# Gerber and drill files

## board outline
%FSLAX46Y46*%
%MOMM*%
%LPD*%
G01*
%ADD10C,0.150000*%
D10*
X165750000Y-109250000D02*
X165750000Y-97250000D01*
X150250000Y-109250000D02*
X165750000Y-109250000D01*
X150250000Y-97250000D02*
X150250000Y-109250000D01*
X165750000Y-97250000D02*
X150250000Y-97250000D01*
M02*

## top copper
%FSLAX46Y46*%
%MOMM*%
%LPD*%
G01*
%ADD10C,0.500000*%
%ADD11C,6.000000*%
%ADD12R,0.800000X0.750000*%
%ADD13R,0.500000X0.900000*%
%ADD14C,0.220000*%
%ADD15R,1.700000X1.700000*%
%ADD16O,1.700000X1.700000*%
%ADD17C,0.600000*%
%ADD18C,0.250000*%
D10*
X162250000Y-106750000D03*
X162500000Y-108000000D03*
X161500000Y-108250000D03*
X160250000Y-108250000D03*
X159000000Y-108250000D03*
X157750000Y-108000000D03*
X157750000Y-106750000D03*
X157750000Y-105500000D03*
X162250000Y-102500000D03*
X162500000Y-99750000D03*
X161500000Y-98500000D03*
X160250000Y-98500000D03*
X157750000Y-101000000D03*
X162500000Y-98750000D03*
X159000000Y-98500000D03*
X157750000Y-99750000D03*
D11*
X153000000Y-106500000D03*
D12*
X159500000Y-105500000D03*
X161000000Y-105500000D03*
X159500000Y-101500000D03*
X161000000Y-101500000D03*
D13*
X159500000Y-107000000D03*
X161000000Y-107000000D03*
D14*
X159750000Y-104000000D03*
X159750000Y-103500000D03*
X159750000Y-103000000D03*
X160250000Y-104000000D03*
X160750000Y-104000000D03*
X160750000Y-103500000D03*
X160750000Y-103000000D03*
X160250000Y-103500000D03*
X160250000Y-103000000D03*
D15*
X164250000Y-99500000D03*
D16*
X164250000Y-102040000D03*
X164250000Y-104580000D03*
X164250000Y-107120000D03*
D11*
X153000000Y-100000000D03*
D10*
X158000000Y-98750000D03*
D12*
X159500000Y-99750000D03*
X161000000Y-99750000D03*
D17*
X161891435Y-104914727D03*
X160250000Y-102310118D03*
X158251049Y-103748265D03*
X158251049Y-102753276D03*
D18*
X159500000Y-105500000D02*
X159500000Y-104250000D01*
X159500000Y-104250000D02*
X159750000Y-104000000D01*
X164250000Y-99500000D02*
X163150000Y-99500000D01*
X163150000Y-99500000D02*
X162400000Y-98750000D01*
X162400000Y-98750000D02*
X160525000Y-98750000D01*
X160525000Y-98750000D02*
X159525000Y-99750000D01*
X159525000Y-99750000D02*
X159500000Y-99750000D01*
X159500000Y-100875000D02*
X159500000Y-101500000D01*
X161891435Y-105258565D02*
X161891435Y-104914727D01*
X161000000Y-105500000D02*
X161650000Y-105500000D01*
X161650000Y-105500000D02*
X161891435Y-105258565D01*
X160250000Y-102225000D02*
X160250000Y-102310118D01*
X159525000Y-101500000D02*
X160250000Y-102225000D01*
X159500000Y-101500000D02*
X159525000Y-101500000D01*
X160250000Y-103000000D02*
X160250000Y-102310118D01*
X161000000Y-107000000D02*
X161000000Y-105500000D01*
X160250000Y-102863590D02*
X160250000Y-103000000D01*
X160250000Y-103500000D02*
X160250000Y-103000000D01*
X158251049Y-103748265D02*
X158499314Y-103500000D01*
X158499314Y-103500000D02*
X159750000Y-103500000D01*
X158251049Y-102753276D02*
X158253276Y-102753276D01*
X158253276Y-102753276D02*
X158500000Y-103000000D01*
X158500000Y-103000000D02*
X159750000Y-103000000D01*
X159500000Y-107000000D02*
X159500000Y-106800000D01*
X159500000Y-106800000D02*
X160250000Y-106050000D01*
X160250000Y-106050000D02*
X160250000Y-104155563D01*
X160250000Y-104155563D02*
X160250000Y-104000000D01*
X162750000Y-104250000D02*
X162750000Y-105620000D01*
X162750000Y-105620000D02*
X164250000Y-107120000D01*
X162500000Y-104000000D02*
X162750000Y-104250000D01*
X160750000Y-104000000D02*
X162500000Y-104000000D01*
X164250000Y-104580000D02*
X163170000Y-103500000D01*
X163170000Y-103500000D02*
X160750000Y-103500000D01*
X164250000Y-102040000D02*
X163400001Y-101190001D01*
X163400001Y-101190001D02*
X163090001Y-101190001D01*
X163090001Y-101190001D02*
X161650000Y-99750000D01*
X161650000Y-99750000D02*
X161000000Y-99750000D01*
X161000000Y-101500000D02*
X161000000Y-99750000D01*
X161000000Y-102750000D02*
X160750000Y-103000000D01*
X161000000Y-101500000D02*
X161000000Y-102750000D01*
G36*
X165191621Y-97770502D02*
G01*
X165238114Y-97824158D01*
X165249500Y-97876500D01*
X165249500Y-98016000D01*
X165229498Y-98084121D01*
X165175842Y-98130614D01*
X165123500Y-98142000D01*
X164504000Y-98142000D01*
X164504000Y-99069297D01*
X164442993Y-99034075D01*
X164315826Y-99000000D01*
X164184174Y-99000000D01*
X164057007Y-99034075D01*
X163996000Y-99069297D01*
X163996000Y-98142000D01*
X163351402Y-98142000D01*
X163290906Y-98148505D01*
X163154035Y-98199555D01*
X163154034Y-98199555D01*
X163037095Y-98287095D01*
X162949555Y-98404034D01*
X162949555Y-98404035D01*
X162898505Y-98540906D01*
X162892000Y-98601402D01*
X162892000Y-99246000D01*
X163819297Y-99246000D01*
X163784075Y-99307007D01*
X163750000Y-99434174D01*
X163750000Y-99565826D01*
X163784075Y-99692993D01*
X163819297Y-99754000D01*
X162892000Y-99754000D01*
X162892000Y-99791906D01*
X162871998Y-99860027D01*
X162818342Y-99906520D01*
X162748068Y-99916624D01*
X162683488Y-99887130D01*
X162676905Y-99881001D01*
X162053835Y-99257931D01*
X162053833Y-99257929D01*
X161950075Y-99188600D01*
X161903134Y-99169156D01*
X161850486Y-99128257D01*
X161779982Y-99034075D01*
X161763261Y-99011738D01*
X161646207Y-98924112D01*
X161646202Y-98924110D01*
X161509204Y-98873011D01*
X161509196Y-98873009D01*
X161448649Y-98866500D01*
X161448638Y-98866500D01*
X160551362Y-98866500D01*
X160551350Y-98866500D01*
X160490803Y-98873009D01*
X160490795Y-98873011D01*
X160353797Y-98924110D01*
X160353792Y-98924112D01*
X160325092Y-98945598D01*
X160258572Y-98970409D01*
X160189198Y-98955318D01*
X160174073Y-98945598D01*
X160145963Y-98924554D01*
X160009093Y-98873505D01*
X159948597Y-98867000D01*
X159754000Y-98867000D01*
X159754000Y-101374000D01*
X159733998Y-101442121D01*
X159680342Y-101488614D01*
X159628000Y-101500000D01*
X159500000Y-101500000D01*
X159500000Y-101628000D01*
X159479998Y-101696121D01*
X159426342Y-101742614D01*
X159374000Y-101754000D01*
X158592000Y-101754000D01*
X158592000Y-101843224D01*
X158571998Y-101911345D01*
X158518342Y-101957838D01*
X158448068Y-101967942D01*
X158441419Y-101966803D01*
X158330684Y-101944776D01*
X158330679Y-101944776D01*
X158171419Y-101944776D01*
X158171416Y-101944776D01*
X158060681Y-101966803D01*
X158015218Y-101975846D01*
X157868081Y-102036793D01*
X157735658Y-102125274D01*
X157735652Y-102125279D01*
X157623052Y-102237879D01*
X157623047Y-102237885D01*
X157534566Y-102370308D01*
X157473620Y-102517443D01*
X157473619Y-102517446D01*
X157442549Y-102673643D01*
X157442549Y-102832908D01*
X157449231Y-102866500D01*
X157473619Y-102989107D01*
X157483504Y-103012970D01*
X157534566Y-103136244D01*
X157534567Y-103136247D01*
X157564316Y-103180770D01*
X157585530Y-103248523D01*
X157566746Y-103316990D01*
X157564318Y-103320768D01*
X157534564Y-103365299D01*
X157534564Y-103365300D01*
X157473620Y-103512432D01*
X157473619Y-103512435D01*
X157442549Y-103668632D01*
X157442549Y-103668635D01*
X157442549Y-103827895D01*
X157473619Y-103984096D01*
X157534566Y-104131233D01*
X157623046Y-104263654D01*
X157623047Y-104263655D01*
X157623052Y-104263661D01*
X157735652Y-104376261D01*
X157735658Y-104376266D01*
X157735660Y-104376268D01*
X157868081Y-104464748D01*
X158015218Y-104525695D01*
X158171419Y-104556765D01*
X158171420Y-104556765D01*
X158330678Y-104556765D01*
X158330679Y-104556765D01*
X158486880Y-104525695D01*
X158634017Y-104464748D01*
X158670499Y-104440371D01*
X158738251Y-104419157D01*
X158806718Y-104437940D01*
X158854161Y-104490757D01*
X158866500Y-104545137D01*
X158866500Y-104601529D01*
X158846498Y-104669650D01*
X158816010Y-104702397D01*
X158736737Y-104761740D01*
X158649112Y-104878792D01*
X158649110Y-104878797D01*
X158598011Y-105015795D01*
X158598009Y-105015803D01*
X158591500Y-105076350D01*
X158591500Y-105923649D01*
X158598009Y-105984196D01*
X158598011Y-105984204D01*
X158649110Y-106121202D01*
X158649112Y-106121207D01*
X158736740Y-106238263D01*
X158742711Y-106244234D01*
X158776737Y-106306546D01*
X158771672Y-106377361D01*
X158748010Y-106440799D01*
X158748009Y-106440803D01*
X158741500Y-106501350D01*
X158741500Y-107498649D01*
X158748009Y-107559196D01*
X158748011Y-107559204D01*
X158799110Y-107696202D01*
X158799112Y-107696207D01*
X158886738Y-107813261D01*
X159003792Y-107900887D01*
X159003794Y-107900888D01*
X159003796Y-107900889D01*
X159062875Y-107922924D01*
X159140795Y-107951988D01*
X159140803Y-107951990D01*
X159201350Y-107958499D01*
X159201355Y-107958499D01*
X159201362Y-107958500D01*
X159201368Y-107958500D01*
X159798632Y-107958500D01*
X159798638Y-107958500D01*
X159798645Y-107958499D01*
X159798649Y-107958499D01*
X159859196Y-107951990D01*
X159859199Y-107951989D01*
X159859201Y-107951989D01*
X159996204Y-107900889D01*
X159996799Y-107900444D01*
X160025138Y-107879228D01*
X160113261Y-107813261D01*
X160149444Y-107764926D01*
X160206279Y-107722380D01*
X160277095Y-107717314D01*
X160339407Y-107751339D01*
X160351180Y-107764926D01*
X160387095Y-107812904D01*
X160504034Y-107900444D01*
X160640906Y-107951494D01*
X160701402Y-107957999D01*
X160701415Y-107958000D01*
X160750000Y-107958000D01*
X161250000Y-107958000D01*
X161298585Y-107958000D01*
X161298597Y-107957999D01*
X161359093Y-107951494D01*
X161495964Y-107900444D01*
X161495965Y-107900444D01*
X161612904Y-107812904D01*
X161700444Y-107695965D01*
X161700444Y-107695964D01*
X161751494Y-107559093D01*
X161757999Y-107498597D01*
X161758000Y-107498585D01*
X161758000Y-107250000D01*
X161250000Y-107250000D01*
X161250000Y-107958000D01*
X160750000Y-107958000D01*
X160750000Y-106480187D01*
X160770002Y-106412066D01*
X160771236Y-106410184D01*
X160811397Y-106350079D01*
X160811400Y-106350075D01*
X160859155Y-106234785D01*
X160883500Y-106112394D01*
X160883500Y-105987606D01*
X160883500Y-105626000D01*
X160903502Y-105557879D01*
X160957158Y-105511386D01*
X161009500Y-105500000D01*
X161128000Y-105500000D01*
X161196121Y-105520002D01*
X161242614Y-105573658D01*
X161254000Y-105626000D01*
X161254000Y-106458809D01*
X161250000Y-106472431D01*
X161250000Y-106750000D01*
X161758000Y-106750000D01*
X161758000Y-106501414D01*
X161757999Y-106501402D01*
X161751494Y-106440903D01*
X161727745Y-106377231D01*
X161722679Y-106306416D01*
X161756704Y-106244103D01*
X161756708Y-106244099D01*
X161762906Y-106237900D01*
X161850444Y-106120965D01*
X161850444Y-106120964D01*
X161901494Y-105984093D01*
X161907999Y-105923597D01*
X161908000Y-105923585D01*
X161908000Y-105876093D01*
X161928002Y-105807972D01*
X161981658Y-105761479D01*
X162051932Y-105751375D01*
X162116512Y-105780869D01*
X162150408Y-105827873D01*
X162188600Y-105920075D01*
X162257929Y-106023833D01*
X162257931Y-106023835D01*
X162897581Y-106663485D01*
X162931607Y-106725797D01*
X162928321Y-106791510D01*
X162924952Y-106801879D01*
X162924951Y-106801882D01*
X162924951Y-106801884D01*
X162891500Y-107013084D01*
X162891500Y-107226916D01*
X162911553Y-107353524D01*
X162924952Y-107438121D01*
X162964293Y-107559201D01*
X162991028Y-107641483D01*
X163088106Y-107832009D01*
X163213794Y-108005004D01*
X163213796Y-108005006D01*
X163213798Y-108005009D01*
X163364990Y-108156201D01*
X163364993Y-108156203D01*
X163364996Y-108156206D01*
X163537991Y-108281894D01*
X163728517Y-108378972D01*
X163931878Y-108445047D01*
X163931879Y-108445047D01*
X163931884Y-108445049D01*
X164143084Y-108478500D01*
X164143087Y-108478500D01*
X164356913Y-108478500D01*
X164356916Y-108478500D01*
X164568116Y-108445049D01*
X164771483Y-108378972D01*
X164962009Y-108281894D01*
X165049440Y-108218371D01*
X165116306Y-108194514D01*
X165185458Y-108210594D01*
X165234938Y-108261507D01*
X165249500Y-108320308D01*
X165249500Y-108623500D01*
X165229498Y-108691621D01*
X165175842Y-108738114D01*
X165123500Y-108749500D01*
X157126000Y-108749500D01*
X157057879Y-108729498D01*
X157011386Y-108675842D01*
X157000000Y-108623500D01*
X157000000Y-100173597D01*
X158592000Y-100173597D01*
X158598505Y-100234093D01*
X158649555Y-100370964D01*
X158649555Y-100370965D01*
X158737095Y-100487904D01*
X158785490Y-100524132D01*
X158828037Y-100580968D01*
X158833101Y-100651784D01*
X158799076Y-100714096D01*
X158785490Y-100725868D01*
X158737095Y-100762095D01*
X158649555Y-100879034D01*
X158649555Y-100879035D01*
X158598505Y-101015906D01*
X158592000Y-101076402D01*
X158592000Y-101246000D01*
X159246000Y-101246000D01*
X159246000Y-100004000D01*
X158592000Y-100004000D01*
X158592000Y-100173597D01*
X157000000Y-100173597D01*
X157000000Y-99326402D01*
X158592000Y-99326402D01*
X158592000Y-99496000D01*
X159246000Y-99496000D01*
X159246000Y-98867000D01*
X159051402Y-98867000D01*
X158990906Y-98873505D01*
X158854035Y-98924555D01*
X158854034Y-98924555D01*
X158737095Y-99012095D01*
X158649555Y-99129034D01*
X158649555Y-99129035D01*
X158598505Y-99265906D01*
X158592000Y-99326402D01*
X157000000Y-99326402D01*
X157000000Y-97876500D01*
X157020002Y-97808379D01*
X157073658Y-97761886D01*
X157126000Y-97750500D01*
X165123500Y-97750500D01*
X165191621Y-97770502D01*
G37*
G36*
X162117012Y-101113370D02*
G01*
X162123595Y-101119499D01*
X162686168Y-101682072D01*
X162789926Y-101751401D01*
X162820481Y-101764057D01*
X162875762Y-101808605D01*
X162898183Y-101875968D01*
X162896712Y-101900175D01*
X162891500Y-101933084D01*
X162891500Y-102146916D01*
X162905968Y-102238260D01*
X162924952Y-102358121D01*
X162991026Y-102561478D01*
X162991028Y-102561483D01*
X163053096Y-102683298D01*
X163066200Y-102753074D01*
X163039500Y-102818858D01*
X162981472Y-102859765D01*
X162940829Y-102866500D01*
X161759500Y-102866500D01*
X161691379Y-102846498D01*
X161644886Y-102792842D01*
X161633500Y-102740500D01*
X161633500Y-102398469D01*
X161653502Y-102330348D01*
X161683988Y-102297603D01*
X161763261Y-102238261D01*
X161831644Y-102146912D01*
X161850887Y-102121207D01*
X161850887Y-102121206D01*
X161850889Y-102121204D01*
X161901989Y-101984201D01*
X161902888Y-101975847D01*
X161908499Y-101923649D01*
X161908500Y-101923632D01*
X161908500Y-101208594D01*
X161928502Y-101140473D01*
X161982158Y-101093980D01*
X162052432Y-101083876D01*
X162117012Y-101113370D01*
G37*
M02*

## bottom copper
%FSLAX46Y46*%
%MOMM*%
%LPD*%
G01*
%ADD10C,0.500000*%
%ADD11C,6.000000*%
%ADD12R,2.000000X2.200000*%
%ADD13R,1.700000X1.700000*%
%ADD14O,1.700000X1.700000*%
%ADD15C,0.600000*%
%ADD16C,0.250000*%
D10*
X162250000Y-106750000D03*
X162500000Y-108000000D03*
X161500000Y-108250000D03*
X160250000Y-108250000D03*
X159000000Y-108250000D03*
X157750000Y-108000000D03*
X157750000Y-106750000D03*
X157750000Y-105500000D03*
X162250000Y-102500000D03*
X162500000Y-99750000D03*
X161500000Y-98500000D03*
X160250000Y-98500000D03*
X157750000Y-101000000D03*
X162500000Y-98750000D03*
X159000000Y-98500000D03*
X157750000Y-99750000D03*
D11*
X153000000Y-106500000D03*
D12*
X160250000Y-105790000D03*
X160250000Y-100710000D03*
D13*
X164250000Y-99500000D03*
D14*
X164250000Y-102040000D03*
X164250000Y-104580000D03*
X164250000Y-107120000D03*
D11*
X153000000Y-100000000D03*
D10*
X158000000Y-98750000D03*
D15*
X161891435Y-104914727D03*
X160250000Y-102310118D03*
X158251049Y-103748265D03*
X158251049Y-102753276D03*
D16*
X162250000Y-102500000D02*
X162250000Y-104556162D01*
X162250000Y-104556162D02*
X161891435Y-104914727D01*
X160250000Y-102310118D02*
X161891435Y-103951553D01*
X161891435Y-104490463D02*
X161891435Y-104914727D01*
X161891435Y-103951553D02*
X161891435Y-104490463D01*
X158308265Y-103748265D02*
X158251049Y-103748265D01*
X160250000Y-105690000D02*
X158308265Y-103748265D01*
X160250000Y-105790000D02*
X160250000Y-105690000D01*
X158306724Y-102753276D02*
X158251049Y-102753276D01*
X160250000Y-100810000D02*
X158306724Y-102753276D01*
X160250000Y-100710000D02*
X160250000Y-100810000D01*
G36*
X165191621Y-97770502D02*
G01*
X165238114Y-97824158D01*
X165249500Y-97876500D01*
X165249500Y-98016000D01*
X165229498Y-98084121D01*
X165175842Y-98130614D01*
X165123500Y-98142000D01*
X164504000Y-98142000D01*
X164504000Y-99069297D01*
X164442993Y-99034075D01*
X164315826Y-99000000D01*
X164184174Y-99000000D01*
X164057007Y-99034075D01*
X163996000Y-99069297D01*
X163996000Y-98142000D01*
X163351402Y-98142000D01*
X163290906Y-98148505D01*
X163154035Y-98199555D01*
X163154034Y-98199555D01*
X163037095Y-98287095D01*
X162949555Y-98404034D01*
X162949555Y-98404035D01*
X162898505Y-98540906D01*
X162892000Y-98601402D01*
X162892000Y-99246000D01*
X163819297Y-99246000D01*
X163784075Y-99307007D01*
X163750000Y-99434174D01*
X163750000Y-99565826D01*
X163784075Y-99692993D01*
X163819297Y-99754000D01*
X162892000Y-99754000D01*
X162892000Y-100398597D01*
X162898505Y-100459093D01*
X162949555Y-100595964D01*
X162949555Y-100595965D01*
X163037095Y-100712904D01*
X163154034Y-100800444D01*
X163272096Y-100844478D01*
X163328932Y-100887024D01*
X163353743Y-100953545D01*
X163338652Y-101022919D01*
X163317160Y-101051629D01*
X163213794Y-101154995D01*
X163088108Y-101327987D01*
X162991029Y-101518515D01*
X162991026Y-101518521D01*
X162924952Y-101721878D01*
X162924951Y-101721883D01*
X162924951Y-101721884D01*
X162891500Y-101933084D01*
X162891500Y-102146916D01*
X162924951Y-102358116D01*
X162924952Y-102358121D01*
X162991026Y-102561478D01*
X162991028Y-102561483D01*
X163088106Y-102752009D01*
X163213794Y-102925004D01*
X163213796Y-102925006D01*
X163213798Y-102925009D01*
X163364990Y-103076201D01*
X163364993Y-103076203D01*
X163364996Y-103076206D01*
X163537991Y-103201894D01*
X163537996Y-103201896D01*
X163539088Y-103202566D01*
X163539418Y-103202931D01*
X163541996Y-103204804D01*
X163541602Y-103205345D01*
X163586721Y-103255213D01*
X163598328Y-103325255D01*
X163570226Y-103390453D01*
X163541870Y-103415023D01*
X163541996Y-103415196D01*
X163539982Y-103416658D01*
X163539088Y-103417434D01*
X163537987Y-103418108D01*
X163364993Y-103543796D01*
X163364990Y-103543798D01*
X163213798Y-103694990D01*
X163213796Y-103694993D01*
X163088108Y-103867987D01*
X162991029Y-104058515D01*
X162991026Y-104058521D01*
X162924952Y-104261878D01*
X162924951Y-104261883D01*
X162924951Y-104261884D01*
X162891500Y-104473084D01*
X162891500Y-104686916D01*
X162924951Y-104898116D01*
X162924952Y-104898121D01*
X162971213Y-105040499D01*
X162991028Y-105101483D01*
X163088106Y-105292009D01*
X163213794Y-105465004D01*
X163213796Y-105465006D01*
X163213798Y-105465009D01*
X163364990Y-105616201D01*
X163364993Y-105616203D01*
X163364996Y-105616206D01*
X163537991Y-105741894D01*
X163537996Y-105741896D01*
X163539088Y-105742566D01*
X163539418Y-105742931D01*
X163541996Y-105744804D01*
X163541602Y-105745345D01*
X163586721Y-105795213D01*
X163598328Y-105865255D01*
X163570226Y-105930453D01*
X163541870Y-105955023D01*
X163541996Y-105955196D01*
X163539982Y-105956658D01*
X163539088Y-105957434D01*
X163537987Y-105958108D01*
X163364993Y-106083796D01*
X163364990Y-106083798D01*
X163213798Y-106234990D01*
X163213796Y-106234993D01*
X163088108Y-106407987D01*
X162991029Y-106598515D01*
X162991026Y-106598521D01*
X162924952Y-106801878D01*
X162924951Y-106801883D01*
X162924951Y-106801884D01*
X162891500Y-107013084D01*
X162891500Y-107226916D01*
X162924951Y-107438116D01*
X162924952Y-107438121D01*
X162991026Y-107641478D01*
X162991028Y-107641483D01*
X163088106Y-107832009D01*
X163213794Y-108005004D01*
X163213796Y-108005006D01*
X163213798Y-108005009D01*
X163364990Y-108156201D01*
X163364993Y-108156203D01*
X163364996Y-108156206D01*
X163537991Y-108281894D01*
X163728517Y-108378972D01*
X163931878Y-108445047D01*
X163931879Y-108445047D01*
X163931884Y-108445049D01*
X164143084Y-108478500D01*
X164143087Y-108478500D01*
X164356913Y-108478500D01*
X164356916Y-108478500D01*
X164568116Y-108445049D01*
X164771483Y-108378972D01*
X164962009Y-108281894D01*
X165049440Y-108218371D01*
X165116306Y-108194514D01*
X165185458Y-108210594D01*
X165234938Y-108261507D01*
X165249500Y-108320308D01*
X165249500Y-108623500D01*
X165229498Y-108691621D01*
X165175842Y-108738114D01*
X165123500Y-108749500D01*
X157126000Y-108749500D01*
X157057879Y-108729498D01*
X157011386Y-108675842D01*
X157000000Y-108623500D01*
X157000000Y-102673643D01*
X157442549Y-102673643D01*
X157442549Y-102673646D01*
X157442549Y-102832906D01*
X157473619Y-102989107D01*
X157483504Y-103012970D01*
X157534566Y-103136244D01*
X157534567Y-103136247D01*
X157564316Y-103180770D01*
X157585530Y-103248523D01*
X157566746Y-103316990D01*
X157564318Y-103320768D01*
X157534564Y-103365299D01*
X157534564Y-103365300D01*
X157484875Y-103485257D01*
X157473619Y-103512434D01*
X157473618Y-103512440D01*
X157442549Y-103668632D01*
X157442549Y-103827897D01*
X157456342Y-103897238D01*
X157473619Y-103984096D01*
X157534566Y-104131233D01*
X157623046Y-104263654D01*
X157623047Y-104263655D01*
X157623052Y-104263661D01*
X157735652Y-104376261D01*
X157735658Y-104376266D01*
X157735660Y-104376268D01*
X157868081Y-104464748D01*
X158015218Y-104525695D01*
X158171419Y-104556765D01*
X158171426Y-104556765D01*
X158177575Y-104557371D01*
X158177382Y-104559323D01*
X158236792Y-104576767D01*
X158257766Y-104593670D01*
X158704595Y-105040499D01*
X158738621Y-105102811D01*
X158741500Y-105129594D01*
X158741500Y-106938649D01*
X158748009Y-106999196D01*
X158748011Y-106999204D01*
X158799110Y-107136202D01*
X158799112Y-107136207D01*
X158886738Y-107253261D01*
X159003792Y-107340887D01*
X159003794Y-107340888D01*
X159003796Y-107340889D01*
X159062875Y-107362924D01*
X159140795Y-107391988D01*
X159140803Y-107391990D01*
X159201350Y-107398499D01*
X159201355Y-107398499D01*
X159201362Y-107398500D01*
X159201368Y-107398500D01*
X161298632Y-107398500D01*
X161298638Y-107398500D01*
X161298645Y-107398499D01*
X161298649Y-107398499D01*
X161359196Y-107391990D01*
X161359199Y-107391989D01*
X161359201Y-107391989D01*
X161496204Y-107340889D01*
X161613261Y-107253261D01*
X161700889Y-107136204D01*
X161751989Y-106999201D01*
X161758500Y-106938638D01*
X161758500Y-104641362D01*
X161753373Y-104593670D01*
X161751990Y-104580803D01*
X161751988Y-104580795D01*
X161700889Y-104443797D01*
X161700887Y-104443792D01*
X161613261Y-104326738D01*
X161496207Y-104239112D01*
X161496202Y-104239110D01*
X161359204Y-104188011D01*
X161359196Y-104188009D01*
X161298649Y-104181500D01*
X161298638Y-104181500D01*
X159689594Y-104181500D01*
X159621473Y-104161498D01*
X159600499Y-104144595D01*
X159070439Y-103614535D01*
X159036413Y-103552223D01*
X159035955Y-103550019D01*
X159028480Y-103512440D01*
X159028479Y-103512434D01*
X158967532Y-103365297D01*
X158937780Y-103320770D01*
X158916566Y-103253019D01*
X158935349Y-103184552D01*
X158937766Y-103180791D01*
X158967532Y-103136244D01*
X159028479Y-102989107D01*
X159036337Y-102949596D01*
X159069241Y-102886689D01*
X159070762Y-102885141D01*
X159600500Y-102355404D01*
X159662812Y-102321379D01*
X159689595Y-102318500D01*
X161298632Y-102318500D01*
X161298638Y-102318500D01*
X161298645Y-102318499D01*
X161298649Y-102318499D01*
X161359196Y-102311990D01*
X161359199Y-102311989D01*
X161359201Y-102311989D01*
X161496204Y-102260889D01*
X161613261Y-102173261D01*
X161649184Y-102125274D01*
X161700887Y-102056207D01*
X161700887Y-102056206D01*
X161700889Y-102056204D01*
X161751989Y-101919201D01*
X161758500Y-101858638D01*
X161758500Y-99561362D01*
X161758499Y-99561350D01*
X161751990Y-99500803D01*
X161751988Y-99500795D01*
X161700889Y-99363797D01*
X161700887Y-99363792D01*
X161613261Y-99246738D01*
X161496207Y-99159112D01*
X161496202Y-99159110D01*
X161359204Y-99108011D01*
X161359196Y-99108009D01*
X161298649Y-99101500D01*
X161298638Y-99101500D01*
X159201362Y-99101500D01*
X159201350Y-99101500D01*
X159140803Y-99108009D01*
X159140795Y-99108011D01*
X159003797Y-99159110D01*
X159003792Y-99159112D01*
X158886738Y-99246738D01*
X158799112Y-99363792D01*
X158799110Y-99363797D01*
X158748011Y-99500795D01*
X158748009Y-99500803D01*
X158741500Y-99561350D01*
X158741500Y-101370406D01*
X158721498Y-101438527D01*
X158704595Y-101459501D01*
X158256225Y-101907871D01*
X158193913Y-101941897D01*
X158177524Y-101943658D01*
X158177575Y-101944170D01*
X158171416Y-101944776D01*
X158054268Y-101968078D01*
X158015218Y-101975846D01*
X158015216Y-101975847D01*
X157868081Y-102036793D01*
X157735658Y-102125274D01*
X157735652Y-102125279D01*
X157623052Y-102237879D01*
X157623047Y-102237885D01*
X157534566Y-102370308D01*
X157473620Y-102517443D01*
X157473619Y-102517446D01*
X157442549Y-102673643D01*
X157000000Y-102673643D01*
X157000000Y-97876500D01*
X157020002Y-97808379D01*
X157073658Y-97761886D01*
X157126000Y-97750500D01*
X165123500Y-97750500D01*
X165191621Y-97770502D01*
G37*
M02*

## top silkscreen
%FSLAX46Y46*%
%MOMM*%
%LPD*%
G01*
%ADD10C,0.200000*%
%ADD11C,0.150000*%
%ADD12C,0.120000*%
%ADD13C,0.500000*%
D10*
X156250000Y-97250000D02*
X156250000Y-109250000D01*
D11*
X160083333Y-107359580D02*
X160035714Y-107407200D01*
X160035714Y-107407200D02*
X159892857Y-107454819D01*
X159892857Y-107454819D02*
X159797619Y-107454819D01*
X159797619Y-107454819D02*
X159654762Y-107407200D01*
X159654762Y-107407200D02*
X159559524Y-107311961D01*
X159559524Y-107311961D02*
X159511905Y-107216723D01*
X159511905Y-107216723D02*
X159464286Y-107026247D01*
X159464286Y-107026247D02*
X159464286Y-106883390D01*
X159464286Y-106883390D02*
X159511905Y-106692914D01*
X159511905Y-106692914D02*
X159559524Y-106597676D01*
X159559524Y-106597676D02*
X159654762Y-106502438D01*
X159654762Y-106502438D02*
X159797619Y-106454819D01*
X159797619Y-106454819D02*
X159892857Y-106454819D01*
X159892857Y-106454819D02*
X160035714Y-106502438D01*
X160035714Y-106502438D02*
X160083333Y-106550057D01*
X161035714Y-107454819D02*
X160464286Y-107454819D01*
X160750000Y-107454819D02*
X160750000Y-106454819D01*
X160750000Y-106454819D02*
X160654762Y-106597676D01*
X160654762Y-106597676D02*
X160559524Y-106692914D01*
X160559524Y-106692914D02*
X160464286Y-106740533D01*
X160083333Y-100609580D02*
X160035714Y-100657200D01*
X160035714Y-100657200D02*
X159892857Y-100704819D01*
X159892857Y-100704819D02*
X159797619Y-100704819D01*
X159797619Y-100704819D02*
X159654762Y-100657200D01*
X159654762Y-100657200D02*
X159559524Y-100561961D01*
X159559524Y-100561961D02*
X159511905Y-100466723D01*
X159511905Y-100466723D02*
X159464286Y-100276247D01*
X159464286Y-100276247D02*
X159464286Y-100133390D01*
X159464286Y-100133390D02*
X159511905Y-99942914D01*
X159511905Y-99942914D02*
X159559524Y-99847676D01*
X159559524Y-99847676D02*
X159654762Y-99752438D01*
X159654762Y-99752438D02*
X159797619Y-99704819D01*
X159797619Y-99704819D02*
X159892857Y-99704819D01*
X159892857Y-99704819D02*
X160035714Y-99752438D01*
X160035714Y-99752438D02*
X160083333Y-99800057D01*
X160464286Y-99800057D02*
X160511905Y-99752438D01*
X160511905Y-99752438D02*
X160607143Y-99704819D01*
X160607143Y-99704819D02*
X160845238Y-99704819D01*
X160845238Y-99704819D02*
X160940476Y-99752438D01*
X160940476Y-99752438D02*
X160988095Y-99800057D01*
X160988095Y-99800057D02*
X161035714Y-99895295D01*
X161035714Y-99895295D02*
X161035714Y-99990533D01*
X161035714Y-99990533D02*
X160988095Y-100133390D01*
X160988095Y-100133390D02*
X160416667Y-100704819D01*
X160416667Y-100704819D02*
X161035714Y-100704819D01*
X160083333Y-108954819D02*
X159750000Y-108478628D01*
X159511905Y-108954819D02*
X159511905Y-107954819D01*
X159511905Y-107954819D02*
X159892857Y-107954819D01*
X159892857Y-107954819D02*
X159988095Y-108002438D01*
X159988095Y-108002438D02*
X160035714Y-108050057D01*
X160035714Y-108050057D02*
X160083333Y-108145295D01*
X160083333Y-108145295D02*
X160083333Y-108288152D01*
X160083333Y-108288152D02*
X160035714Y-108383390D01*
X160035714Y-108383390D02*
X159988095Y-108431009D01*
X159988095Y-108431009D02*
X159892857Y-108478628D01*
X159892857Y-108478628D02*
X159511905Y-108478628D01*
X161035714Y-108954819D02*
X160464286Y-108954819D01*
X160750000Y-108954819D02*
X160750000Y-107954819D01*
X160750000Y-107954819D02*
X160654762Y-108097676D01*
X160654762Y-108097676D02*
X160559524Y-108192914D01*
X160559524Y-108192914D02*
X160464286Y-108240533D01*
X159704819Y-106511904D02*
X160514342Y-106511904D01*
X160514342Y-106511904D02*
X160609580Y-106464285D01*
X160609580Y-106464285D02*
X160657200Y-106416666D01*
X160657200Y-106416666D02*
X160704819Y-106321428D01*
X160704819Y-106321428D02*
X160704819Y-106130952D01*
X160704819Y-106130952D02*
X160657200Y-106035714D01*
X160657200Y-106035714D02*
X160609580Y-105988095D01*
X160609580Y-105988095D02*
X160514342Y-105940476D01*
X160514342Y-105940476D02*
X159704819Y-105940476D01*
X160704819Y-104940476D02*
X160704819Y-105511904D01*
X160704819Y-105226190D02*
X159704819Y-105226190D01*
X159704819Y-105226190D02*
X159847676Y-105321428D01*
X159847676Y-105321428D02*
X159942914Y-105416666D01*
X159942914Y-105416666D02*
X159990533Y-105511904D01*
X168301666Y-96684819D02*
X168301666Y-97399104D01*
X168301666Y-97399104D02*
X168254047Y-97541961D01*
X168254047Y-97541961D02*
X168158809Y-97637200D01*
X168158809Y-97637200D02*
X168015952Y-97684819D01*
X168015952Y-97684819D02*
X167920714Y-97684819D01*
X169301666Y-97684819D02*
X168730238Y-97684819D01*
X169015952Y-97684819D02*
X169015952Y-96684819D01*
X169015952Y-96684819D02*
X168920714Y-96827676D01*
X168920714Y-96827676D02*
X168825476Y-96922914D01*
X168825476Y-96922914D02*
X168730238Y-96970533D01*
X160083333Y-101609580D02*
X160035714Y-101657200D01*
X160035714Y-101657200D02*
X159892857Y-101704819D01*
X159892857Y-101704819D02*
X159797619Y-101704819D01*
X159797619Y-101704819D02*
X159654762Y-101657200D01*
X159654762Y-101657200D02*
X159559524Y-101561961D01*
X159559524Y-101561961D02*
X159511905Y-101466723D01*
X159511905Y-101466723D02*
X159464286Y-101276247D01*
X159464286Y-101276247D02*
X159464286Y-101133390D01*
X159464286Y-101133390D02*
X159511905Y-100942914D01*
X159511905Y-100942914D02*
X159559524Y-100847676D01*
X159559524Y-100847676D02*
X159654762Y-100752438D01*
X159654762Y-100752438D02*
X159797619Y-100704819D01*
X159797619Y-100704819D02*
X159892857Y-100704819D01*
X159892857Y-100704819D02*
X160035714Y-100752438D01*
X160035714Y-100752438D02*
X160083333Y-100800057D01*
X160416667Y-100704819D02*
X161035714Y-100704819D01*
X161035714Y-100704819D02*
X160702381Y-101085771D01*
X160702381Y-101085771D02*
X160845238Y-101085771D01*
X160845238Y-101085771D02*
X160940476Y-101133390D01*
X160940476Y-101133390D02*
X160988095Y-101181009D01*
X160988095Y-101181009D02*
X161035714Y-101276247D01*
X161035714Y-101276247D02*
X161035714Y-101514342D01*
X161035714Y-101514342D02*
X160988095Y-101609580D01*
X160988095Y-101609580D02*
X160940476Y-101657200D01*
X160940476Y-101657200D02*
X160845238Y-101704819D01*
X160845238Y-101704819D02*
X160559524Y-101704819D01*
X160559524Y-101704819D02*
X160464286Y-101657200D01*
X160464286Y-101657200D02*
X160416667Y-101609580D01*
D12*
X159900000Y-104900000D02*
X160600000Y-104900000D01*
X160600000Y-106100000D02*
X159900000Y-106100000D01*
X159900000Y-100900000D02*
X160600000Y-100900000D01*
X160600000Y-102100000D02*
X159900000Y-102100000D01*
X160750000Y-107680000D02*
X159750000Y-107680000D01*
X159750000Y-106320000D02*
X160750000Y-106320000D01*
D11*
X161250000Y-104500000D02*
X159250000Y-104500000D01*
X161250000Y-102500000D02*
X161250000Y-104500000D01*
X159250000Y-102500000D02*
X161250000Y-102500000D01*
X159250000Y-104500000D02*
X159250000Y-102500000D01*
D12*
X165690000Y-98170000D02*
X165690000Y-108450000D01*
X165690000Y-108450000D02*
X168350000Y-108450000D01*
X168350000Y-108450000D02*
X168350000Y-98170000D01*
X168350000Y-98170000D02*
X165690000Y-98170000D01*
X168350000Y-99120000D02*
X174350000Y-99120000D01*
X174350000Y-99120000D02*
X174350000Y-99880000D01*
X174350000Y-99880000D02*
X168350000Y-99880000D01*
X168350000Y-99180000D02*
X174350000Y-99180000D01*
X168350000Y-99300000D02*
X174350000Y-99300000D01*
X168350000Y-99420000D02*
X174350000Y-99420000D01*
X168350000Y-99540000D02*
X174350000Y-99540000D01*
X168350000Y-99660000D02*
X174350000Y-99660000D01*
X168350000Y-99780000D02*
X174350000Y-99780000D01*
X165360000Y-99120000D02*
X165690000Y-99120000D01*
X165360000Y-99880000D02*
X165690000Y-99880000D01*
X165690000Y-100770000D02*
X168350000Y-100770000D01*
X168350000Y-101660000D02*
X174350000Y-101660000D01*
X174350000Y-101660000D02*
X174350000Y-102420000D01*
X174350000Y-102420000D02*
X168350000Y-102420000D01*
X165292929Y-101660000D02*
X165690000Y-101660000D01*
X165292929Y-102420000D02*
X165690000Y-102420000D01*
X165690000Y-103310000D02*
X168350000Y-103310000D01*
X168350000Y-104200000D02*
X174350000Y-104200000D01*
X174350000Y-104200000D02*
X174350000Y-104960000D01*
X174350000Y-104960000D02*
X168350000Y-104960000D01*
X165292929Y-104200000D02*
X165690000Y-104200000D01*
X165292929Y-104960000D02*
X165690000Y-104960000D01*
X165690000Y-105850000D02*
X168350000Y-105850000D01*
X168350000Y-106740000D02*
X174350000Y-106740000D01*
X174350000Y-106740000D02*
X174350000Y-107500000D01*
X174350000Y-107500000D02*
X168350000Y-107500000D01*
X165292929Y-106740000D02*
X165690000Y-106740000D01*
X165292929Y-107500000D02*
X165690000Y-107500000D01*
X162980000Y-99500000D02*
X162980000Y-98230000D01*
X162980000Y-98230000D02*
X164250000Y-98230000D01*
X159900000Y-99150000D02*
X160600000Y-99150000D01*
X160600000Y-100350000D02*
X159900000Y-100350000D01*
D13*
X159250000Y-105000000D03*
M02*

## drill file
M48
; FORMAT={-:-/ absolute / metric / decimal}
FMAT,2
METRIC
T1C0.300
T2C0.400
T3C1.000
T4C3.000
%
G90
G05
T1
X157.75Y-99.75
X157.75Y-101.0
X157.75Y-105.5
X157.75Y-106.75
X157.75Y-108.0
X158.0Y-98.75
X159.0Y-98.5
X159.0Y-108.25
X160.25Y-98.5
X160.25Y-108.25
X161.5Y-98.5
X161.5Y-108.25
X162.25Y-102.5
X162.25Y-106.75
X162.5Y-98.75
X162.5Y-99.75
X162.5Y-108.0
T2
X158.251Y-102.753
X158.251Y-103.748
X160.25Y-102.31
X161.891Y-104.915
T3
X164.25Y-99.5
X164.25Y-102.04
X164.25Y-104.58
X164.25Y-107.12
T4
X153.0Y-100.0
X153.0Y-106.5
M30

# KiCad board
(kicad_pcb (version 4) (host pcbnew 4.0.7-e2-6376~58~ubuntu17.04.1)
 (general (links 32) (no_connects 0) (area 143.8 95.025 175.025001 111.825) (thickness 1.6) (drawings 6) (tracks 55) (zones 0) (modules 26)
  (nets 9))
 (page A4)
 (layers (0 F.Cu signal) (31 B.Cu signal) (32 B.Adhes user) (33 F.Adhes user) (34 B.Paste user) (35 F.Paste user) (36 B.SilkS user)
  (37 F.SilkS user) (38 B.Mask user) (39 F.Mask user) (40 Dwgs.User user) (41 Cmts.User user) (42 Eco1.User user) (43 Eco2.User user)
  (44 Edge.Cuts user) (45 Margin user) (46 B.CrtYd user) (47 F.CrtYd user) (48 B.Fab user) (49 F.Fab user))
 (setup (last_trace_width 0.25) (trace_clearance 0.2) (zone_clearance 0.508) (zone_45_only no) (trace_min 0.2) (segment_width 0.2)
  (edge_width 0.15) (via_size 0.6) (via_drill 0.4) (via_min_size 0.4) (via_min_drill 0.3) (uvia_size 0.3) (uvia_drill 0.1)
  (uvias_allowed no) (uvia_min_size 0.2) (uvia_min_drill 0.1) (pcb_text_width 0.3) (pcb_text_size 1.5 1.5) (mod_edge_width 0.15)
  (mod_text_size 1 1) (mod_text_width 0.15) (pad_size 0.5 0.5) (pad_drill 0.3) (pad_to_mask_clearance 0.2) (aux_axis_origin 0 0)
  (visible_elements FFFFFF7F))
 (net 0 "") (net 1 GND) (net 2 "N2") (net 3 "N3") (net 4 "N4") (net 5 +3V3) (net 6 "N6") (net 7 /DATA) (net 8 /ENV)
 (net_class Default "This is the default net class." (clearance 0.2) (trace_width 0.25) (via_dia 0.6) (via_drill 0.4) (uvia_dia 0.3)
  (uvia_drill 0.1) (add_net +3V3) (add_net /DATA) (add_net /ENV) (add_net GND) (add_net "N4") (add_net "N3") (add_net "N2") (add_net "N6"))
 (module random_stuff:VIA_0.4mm (layer F.Cu) (at 162.25 106.75)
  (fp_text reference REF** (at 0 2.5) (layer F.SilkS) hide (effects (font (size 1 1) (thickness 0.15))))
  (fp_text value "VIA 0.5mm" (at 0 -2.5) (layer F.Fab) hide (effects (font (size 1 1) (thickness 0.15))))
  (pad 1 thru_hole circle (at 0 0) (size 0.5 0.5) (drill 0.3) (layers *.Cu) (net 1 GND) (zone_connect 2)))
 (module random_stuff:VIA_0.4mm (layer F.Cu) (at 162.5 108)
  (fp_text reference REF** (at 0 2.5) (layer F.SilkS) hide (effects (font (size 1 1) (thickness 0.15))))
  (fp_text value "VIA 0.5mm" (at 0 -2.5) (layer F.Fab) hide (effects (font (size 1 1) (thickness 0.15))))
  (pad 1 thru_hole circle (at 0 0) (size 0.5 0.5) (drill 0.3) (layers *.Cu) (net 1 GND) (zone_connect 2)))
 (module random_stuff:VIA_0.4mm (layer F.Cu) (at 161.5 108.25)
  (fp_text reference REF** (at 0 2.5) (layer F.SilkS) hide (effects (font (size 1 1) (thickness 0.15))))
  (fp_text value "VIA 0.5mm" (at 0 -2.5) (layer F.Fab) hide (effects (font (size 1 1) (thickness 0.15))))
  (pad 1 thru_hole circle (at 0 0) (size 0.5 0.5) (drill 0.3) (layers *.Cu) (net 1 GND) (zone_connect 2)))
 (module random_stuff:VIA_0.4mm (layer F.Cu) (at 160.25 108.25)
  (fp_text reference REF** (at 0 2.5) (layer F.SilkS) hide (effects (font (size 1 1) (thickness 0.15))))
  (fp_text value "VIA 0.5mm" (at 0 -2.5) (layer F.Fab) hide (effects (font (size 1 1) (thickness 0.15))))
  (pad 1 thru_hole circle (at 0 0) (size 0.5 0.5) (drill 0.3) (layers *.Cu) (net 1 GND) (zone_connect 2)))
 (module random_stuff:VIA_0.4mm (layer F.Cu) (at 159 108.25)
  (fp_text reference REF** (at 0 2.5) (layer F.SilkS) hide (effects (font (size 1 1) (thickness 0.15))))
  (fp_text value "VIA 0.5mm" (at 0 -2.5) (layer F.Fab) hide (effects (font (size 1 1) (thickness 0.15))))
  (pad 1 thru_hole circle (at 0 0) (size 0.5 0.5) (drill 0.3) (layers *.Cu) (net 1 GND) (zone_connect 2)))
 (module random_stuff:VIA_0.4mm (layer F.Cu) (at 157.75 108)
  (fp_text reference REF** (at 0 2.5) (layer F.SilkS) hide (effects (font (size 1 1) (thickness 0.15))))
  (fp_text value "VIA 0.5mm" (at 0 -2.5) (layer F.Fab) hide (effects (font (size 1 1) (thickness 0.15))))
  (pad 1 thru_hole circle (at 0 0) (size 0.5 0.5) (drill 0.3) (layers *.Cu) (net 1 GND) (zone_connect 2)))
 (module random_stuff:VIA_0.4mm (layer F.Cu) (at 157.75 106.75)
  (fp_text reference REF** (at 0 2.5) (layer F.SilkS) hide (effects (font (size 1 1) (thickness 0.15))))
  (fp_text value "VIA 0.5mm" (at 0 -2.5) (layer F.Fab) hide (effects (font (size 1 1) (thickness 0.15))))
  (pad 1 thru_hole circle (at 0 0) (size 0.5 0.5) (drill 0.3) (layers *.Cu) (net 1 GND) (zone_connect 2)))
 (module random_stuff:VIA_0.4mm (layer F.Cu) (at 157.75 105.5)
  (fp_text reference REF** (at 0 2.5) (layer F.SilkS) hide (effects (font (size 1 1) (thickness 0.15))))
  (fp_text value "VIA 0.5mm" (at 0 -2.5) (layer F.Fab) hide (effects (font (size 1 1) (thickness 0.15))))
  (pad 1 thru_hole circle (at 0 0) (size 0.5 0.5) (drill 0.3) (layers *.Cu) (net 1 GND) (zone_connect 2)))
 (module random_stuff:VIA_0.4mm (layer F.Cu) (at 162.25 102.5)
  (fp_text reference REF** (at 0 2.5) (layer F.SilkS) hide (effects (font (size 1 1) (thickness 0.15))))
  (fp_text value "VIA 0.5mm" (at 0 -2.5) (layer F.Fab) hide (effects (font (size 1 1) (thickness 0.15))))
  (pad 1 thru_hole circle (at 0 0) (size 0.5 0.5) (drill 0.3) (layers *.Cu) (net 1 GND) (zone_connect 2)))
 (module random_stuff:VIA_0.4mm (layer F.Cu) (at 162.5 99.75)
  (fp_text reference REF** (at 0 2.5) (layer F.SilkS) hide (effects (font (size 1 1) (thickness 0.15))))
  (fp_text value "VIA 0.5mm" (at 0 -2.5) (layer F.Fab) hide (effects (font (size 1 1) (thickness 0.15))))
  (pad 1 thru_hole circle (at 0 0) (size 0.5 0.5) (drill 0.3) (layers *.Cu) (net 1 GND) (zone_connect 2)))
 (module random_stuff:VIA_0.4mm (layer F.Cu) (at 161.5 98.5)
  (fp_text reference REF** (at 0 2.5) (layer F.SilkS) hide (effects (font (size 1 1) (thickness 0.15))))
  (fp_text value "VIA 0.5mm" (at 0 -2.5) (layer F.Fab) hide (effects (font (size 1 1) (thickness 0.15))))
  (pad 1 thru_hole circle (at 0 0) (size 0.5 0.5) (drill 0.3) (layers *.Cu) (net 1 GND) (zone_connect 2)))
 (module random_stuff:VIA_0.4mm (layer F.Cu) (at 160.25 98.5)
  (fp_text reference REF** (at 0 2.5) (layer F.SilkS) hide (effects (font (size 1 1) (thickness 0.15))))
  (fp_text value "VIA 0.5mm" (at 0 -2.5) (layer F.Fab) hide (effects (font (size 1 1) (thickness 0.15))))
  (pad 1 thru_hole circle (at 0 0) (size 0.5 0.5) (drill 0.3) (layers *.Cu) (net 1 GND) (zone_connect 2)))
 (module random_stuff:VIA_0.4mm (layer F.Cu) (at 157.75 101)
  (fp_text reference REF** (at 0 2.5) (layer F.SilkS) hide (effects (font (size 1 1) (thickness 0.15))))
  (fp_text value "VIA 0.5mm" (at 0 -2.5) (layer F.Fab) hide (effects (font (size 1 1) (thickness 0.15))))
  (pad 1 thru_hole circle (at 0 0) (size 0.5 0.5) (drill 0.3) (layers *.Cu) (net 1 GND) (zone_connect 2)))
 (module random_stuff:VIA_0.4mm (layer F.Cu) (at 162.5 98.75)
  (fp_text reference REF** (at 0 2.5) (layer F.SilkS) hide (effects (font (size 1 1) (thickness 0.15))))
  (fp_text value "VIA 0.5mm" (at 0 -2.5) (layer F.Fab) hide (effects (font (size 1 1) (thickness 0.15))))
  (pad 1 thru_hole circle (at 0 0) (size 0.5 0.5) (drill 0.3) (layers *.Cu) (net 1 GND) (zone_connect 2)))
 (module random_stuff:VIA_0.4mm (layer F.Cu) (at 159 98.5)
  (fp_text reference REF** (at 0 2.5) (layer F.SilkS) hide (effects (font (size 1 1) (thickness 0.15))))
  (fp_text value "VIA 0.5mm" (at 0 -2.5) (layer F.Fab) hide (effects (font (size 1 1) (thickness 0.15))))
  (pad 1 thru_hole circle (at 0 0) (size 0.5 0.5) (drill 0.3) (layers *.Cu) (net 1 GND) (zone_connect 2)))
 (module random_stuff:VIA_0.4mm (layer F.Cu) (at 157.75 99.75)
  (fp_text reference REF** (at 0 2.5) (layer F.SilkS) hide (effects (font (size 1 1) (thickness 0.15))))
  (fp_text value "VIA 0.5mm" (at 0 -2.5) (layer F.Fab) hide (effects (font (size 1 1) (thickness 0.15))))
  (pad 1 thru_hole circle (at 0 0) (size 0.5 0.5) (drill 0.3) (layers *.Cu) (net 1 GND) (zone_connect 2)))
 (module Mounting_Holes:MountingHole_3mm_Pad (layer F.Cu) (at 153 106.5)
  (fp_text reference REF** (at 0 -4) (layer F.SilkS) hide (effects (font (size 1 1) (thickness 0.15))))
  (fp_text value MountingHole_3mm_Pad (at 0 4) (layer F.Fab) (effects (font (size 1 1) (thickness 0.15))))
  (pad 1 thru_hole circle (at 0 0) (size 6 6) (drill 3) (layers *.Cu *.Mask)))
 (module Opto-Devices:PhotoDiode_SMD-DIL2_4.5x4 (layer B.Cu) (at 160.25 103.25 270)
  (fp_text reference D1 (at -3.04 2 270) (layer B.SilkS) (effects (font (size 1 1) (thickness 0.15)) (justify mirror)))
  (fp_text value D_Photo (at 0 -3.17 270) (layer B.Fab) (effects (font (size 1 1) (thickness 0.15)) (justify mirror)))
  (pad 2 smd rect (at 2.54 0 90) (size 2.2 2) (layers B.Cu B.Paste B.Mask) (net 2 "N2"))
  (pad 1 smd rect (at -2.54 0 90) (size 2.2 2) (layers B.Cu B.Paste B.Mask) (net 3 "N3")))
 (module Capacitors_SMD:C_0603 (layer F.Cu) (at 160.25 105.5 180)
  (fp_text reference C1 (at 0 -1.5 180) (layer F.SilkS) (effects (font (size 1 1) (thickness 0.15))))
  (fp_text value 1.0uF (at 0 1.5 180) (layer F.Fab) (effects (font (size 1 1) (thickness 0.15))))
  (fp_line (start 0.35 0.6) (end -0.35 0.6) (layer F.SilkS) (width 0.12))
  (fp_line (start -0.35 -0.6) (end 0.35 -0.6) (layer F.SilkS) (width 0.12))
  (pad 2 smd rect (at 0.75 0 180) (size 0.8 0.75) (layers F.Cu F.Paste F.Mask) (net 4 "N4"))
  (pad 1 smd rect (at -0.75 0 180) (size 0.8 0.75) (layers F.Cu F.Paste F.Mask) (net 1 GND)))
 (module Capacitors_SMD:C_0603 (layer F.Cu) (at 160.25 101.5 180)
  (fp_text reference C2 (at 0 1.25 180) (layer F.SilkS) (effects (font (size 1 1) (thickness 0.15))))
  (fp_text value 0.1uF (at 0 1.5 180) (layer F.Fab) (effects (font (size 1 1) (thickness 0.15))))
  (fp_line (start 0.35 0.6) (end -0.35 0.6) (layer F.SilkS) (width 0.12))
  (fp_line (start -0.35 -0.6) (end 0.35 -0.6) (layer F.SilkS) (width 0.12))
  (pad 2 smd rect (at 0.75 0 180) (size 0.8 0.75) (layers F.Cu F.Paste F.Mask) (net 1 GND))
  (pad 1 smd rect (at -0.75 0 180) (size 0.8 0.75) (layers F.Cu F.Paste F.Mask) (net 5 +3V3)))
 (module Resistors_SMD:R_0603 (layer F.Cu) (at 160.25 107)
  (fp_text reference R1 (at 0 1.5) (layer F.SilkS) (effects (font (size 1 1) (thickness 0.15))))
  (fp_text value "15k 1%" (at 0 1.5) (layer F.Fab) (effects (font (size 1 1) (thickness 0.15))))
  (fp_line (start 0.5 0.68) (end -0.5 0.68) (layer F.SilkS) (width 0.12))
  (fp_line (start -0.5 -0.68) (end 0.5 -0.68) (layer F.SilkS) (width 0.12))
  (pad 1 smd rect (at -0.75 0) (size 0.5 0.9) (layers F.Cu F.Paste F.Mask) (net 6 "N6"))
  (pad 2 smd rect (at 0.75 0) (size 0.5 0.9) (layers F.Cu F.Paste F.Mask) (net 1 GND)))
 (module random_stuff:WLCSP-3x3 (layer F.Cu) (at 160.25 103.5 90)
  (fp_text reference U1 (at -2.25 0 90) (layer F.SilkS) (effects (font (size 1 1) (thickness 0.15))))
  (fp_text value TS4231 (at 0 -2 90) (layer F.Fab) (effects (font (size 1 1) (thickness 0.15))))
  (fp_line (start -1 1) (end -1 -1) (layer F.SilkS) (width 0.15))
  (fp_line (start 1 1) (end -1 1) (layer F.SilkS) (width 0.15))
  (fp_line (start 1 -1) (end 1 1) (layer F.SilkS) (width 0.15))
  (fp_line (start -1 -1) (end 1 -1) (layer F.SilkS) (width 0.15))
  (pad A1 smd circle (at -0.5 -0.5 90) (size 0.22 0.22) (layers F.Cu F.Paste F.Mask) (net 4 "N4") (solder_mask_margin 0.05))
  (pad A2 smd circle (at 0 -0.5 90) (size 0.22 0.22) (layers F.Cu F.Paste F.Mask) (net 2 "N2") (solder_mask_margin 0.05))
  (pad A3 smd circle (at 0.5 -0.5 90) (size 0.22 0.22) (layers F.Cu F.Paste F.Mask) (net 3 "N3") (solder_mask_margin 0.05))
  (pad B1 smd circle (at -0.5 0 90) (size 0.22 0.22) (layers F.Cu F.Paste F.Mask) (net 6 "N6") (solder_mask_margin 0.05))
  (pad C1 smd circle (at -0.5 0.5 90) (size 0.22 0.22) (layers F.Cu F.Paste F.Mask) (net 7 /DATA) (solder_mask_margin 0.05))
  (pad C2 smd circle (at 0 0.5 90) (size 0.22 0.22) (layers F.Cu F.Paste F.Mask) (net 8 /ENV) (solder_mask_margin 0.05))
  (pad C3 smd circle (at 0.5 0.5 90) (size 0.22 0.22) (layers F.Cu F.Paste F.Mask) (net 5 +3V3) (solder_mask_margin 0.05))
  (pad B2 smd circle (at 0 0 90) (size 0.22 0.22) (layers F.Cu F.Paste F.Mask) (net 1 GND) (solder_mask_margin 0.05))
  (pad B3 smd circle (at 0.5 0 90) (size 0.22 0.22) (layers F.Cu F.Paste F.Mask) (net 1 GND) (solder_mask_margin 0.05))
  (pad "" smd circle (at -1.5 -1 90) (size 0.5 0.5) (layers F.SilkS)))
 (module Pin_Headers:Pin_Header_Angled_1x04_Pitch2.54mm (layer F.Cu) (at 164.25 99.5)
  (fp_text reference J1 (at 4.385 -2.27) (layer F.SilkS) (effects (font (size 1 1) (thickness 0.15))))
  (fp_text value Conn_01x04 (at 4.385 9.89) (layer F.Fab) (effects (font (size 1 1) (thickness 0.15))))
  (fp_line (start 1.44 -1.33) (end 1.44 8.95) (layer F.SilkS) (width 0.12))
  (fp_line (start 1.44 8.95) (end 4.1 8.95) (layer F.SilkS) (width 0.12))
  (fp_line (start 4.1 8.95) (end 4.1 -1.33) (layer F.SilkS) (width 0.12))
  (fp_line (start 4.1 -1.33) (end 1.44 -1.33) (layer F.SilkS) (width 0.12))
  (fp_line (start 4.1 -0.38) (end 10.1 -0.38) (layer F.SilkS) (width 0.12))
  (fp_line (start 10.1 -0.38) (end 10.1 0.38) (layer F.SilkS) (width 0.12))
  (fp_line (start 10.1 0.38) (end 4.1 0.38) (layer F.SilkS) (width 0.12))
  (fp_line (start 4.1 -0.32) (end 10.1 -0.32) (layer F.SilkS) (width 0.12))
  (fp_line (start 4.1 -0.2) (end 10.1 -0.2) (layer F.SilkS) (width 0.12))
  (fp_line (start 4.1 -0.08) (end 10.1 -0.08) (layer F.SilkS) (width 0.12))
  (fp_line (start 4.1 0.04) (end 10.1 0.04) (layer F.SilkS) (width 0.12))
  (fp_line (start 4.1 0.16) (end 10.1 0.16) (layer F.SilkS) (width 0.12))
  (fp_line (start 4.1 0.28) (end 10.1 0.28) (layer F.SilkS) (width 0.12))
  (fp_line (start 1.11 -0.38) (end 1.44 -0.38) (layer F.SilkS) (width 0.12))
  (fp_line (start 1.11 0.38) (end 1.44 0.38) (layer F.SilkS) (width 0.12))
  (fp_line (start 1.44 1.27) (end 4.1 1.27) (layer F.SilkS) (width 0.12))
  (fp_line (start 4.1 2.16) (end 10.1 2.16) (layer F.SilkS) (width 0.12))
  (fp_line (start 10.1 2.16) (end 10.1 2.92) (layer F.SilkS) (width 0.12))
  (fp_line (start 10.1 2.92) (end 4.1 2.92) (layer F.SilkS) (width 0.12))
  (fp_line (start 1.042929 2.16) (end 1.44 2.16) (layer F.SilkS) (width 0.12))
  (fp_line (start 1.042929 2.92) (end 1.44 2.92) (layer F.SilkS) (width 0.12))
  (fp_line (start 1.44 3.81) (end 4.1 3.81) (layer F.SilkS) (width 0.12))
  (fp_line (start 4.1 4.7) (end 10.1 4.7) (layer F.SilkS) (width 0.12))
  (fp_line (start 10.1 4.7) (end 10.1 5.46) (layer F.SilkS) (width 0.12))
  (fp_line (start 10.1 5.46) (end 4.1 5.46) (layer F.SilkS) (width 0.12))
  (fp_line (start 1.042929 4.7) (end 1.44 4.7) (layer F.SilkS) (width 0.12))
  (fp_line (start 1.042929 5.46) (end 1.44 5.46) (layer F.SilkS) (width 0.12))
  (fp_line (start 1.44 6.35) (end 4.1 6.35) (layer F.SilkS) (width 0.12))
  (fp_line (start 4.1 7.24) (end 10.1 7.24) (layer F.SilkS) (width 0.12))
  (fp_line (start 10.1 7.24) (end 10.1 8) (layer F.SilkS) (width 0.12))
  (fp_line (start 10.1 8) (end 4.1 8) (layer F.SilkS) (width 0.12))
  (fp_line (start 1.042929 7.24) (end 1.44 7.24) (layer F.SilkS) (width 0.12))
  (fp_line (start 1.042929 8) (end 1.44 8) (layer F.SilkS) (width 0.12))
  (fp_line (start -1.27 0) (end -1.27 -1.27) (layer F.SilkS) (width 0.12))
  (fp_line (start -1.27 -1.27) (end 0 -1.27) (layer F.SilkS) (width 0.12))
  (pad 1 thru_hole rect (at 0 0) (size 1.7 1.7) (drill 1) (layers *.Cu *.Mask) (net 1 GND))
  (pad 2 thru_hole oval (at 0 2.54) (size 1.7 1.7) (drill 1) (layers *.Cu *.Mask) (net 5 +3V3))
  (pad 3 thru_hole oval (at 0 5.08) (size 1.7 1.7) (drill 1) (layers *.Cu *.Mask) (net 8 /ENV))
  (pad 4 thru_hole oval (at 0 7.62) (size 1.7 1.7) (drill 1) (layers *.Cu *.Mask) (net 7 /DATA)))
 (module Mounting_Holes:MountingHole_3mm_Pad (layer F.Cu) (at 153 100)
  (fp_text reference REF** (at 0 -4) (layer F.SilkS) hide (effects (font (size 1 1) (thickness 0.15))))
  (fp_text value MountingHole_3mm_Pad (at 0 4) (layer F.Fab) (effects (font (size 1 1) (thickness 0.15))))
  (pad 1 thru_hole circle (at 0 0) (size 6 6) (drill 3) (layers *.Cu *.Mask)))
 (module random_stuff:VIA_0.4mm (layer F.Cu) (at 158 98.75)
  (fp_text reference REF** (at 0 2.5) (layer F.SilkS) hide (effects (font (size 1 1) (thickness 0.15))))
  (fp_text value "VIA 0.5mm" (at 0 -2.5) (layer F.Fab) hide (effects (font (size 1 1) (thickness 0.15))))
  (pad 1 thru_hole circle (at 0 0) (size 0.5 0.5) (drill 0.3) (layers *.Cu) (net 1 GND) (zone_connect 2)))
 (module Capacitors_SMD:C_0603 (layer F.Cu) (at 160.25 99.75 180)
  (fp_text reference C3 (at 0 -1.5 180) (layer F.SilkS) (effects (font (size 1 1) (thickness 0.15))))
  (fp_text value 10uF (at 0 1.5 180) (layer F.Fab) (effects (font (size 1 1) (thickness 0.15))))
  (fp_line (start 0.35 0.6) (end -0.35 0.6) (layer F.SilkS) (width 0.12))
  (fp_line (start -0.35 -0.6) (end 0.35 -0.6) (layer F.SilkS) (width 0.12))
  (pad 2 smd rect (at 0.75 0 180) (size 0.8 0.75) (layers F.Cu F.Paste F.Mask) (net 1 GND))
  (pad 1 smd rect (at -0.75 0 180) (size 0.8 0.75) (layers F.Cu F.Paste F.Mask) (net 5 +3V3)))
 (gr_line (start 156.25 97.25) (end 156.25 109.25) (layer F.SilkS) (width 0.2))
 (gr_line (start 165.75 109.25) (end 165.75 97.25) (layer Edge.Cuts) (width 0.15))
 (gr_line (start 150.25 109.25) (end 165.75 109.25) (layer Edge.Cuts) (width 0.15))
 (gr_line (start 150.25 97.25) (end 150.25 109.25) (layer Edge.Cuts) (width 0.15))
 (gr_line (start 165.75 97.25) (end 150.25 97.25) (layer Edge.Cuts) (width 0.15))
 (segment (start 159.5 105.5) (end 159.5 104.25) (width 0.25) (layer F.Cu) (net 4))
 (segment (start 159.5 104.25) (end 159.75 104) (width 0.25) (layer F.Cu) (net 4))
 (segment (start 162.25 102.5) (end 162.25 104.556162) (width 0.25) (layer B.Cu) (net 1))
 (segment (start 162.25 104.556162) (end 161.891435 104.914727) (width 0.25) (layer B.Cu) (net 1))
 (segment (start 164.25 99.5) (end 163.15 99.5) (width 0.25) (layer F.Cu) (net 1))
 (segment (start 163.15 99.5) (end 162.4 98.75) (width 0.25) (layer F.Cu) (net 1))
 (segment (start 162.4 98.75) (end 160.525 98.75) (width 0.25) (layer F.Cu) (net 1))
 (segment (start 160.525 98.75) (end 159.525 99.75) (width 0.25) (layer F.Cu) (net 1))
 (segment (start 159.525 99.75) (end 159.5 99.75) (width 0.25) (layer F.Cu) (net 1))
 (segment (start 159.5 100.875) (end 159.5 101.5) (width 0.25) (layer F.Cu) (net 1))
 (segment (start 161.891435 105.258565) (end 161.891435 104.914727) (width 0.25) (layer F.Cu) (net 1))
 (segment (start 161 105.5) (end 161.65 105.5) (width 0.25) (layer F.Cu) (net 1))
 (segment (start 161.65 105.5) (end 161.891435 105.258565) (width 0.25) (layer F.Cu) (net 1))
 (segment (start 160.25 102.310118) (end 161.891435 103.951553) (width 0.25) (layer B.Cu) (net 1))
 (via (at 161.891435 104.914727) (size 0.6) (drill 0.4) (layers F.Cu B.Cu) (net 1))
 (segment (start 161.891435 104.490463) (end 161.891435 104.914727) (width 0.25) (layer B.Cu) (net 1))
 (segment (start 161.891435 103.951553) (end 161.891435 104.490463) (width 0.25) (layer B.Cu) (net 1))
 (segment (start 160.25 102.225) (end 160.25 102.310118) (width 0.25) (layer F.Cu) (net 1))
 (segment (start 159.525 101.5) (end 160.25 102.225) (width 0.25) (layer F.Cu) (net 1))
 (segment (start 159.5 101.5) (end 159.525 101.5) (width 0.25) (layer F.Cu) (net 1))
 (via (at 160.25 102.310118) (size 0.6) (drill 0.4) (layers F.Cu B.Cu) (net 1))
 (segment (start 160.25 103) (end 160.25 102.310118) (width 0.25) (layer F.Cu) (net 1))
 (segment (start 161 107) (end 161 105.5) (width 0.25) (layer F.Cu) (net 1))
 (segment (start 160.25 102.86359) (end 160.25 103) (width 0.25) (layer F.Cu) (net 1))
 (segment (start 160.25 103.5) (end 160.25 103) (width 0.25) (layer F.Cu) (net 1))
 (segment (start 158.251049 103.748265) (end 158.499314 103.5) (width 0.25) (layer F.Cu) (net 2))
 (segment (start 158.499314 103.5) (end 159.75 103.5) (width 0.25) (layer F.Cu) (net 2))
 (segment (start 158.308265 103.748265) (end 158.251049 103.748265) (width 0.25) (layer B.Cu) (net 2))
 (segment (start 160.25 105.69) (end 158.308265 103.748265) (width 0.25) (layer B.Cu) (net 2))
 (segment (start 160.25 105.79) (end 160.25 105.69) (width 0.25) (layer B.Cu) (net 2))
 (via (at 158.251049 103.748265) (size 0.6) (drill 0.4) (layers F.Cu B.Cu) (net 2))
 (segment (start 158.251049 102.753276) (end 158.253276 102.753276) (width 0.25) (layer F.Cu) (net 3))
 (segment (start 158.253276 102.753276) (end 158.5 103) (width 0.25) (layer F.Cu) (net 3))
 (segment (start 158.5 103) (end 159.75 103) (width 0.25) (layer F.Cu) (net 3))
 (segment (start 158.306724 102.753276) (end 158.251049 102.753276) (width 0.25) (layer B.Cu) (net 3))
 (segment (start 160.25 100.81) (end 158.306724 102.753276) (width 0.25) (layer B.Cu) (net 3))
 (segment (start 160.25 100.71) (end 160.25 100.81) (width 0.25) (layer B.Cu) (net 3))
 (via (at 158.251049 102.753276) (size 0.6) (drill 0.4) (layers F.Cu B.Cu) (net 3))
 (segment (start 159.5 107) (end 159.5 106.8) (width 0.25) (layer F.Cu) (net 6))
 (segment (start 159.5 106.8) (end 160.25 106.05) (width 0.25) (layer F.Cu) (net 6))
 (segment (start 160.25 106.05) (end 160.25 104.155563) (width 0.25) (layer F.Cu) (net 6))
 (segment (start 160.25 104.155563) (end 160.25 104) (width 0.25) (layer F.Cu) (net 6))
 (segment (start 162.75 104.25) (end 162.75 105.62) (width 0.25) (layer F.Cu) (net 7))
 (segment (start 162.75 105.62) (end 164.25 107.12) (width 0.25) (layer F.Cu) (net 7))
 (segment (start 162.5 104) (end 162.75 104.25) (width 0.25) (layer F.Cu) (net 7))
 (segment (start 160.75 104) (end 162.5 104) (width 0.25) (layer F.Cu) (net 7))
 (segment (start 164.25 104.58) (end 163.17 103.5) (width 0.25) (layer F.Cu) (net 8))
 (segment (start 163.17 103.5) (end 160.75 103.5) (width 0.25) (layer F.Cu) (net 8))
 (segment (start 164.25 102.04) (end 163.400001 101.190001) (width 0.25) (layer F.Cu) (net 5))
 (segment (start 163.400001 101.190001) (end 163.090001 101.190001) (width 0.25) (layer F.Cu) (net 5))
 (segment (start 163.090001 101.190001) (end 161.65 99.75) (width 0.25) (layer F.Cu) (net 5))
 (segment (start 161.65 99.75) (end 161 99.75) (width 0.25) (layer F.Cu) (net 5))
 (segment (start 161 101.5) (end 161 99.75) (width 0.25) (layer F.Cu) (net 5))
 (segment (start 161 102.75) (end 160.75 103) (width 0.25) (layer F.Cu) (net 5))
 (segment (start 161 101.5) (end 161 102.75) (width 0.25) (layer F.Cu) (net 5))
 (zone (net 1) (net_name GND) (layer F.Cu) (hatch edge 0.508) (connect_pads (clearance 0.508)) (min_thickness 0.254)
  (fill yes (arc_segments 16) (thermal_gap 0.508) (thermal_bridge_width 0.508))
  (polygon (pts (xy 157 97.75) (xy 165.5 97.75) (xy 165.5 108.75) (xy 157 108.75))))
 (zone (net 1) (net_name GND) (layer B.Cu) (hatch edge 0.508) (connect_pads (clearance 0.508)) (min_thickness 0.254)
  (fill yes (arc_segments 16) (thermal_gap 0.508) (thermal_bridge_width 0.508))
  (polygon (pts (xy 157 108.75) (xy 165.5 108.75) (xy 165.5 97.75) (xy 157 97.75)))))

